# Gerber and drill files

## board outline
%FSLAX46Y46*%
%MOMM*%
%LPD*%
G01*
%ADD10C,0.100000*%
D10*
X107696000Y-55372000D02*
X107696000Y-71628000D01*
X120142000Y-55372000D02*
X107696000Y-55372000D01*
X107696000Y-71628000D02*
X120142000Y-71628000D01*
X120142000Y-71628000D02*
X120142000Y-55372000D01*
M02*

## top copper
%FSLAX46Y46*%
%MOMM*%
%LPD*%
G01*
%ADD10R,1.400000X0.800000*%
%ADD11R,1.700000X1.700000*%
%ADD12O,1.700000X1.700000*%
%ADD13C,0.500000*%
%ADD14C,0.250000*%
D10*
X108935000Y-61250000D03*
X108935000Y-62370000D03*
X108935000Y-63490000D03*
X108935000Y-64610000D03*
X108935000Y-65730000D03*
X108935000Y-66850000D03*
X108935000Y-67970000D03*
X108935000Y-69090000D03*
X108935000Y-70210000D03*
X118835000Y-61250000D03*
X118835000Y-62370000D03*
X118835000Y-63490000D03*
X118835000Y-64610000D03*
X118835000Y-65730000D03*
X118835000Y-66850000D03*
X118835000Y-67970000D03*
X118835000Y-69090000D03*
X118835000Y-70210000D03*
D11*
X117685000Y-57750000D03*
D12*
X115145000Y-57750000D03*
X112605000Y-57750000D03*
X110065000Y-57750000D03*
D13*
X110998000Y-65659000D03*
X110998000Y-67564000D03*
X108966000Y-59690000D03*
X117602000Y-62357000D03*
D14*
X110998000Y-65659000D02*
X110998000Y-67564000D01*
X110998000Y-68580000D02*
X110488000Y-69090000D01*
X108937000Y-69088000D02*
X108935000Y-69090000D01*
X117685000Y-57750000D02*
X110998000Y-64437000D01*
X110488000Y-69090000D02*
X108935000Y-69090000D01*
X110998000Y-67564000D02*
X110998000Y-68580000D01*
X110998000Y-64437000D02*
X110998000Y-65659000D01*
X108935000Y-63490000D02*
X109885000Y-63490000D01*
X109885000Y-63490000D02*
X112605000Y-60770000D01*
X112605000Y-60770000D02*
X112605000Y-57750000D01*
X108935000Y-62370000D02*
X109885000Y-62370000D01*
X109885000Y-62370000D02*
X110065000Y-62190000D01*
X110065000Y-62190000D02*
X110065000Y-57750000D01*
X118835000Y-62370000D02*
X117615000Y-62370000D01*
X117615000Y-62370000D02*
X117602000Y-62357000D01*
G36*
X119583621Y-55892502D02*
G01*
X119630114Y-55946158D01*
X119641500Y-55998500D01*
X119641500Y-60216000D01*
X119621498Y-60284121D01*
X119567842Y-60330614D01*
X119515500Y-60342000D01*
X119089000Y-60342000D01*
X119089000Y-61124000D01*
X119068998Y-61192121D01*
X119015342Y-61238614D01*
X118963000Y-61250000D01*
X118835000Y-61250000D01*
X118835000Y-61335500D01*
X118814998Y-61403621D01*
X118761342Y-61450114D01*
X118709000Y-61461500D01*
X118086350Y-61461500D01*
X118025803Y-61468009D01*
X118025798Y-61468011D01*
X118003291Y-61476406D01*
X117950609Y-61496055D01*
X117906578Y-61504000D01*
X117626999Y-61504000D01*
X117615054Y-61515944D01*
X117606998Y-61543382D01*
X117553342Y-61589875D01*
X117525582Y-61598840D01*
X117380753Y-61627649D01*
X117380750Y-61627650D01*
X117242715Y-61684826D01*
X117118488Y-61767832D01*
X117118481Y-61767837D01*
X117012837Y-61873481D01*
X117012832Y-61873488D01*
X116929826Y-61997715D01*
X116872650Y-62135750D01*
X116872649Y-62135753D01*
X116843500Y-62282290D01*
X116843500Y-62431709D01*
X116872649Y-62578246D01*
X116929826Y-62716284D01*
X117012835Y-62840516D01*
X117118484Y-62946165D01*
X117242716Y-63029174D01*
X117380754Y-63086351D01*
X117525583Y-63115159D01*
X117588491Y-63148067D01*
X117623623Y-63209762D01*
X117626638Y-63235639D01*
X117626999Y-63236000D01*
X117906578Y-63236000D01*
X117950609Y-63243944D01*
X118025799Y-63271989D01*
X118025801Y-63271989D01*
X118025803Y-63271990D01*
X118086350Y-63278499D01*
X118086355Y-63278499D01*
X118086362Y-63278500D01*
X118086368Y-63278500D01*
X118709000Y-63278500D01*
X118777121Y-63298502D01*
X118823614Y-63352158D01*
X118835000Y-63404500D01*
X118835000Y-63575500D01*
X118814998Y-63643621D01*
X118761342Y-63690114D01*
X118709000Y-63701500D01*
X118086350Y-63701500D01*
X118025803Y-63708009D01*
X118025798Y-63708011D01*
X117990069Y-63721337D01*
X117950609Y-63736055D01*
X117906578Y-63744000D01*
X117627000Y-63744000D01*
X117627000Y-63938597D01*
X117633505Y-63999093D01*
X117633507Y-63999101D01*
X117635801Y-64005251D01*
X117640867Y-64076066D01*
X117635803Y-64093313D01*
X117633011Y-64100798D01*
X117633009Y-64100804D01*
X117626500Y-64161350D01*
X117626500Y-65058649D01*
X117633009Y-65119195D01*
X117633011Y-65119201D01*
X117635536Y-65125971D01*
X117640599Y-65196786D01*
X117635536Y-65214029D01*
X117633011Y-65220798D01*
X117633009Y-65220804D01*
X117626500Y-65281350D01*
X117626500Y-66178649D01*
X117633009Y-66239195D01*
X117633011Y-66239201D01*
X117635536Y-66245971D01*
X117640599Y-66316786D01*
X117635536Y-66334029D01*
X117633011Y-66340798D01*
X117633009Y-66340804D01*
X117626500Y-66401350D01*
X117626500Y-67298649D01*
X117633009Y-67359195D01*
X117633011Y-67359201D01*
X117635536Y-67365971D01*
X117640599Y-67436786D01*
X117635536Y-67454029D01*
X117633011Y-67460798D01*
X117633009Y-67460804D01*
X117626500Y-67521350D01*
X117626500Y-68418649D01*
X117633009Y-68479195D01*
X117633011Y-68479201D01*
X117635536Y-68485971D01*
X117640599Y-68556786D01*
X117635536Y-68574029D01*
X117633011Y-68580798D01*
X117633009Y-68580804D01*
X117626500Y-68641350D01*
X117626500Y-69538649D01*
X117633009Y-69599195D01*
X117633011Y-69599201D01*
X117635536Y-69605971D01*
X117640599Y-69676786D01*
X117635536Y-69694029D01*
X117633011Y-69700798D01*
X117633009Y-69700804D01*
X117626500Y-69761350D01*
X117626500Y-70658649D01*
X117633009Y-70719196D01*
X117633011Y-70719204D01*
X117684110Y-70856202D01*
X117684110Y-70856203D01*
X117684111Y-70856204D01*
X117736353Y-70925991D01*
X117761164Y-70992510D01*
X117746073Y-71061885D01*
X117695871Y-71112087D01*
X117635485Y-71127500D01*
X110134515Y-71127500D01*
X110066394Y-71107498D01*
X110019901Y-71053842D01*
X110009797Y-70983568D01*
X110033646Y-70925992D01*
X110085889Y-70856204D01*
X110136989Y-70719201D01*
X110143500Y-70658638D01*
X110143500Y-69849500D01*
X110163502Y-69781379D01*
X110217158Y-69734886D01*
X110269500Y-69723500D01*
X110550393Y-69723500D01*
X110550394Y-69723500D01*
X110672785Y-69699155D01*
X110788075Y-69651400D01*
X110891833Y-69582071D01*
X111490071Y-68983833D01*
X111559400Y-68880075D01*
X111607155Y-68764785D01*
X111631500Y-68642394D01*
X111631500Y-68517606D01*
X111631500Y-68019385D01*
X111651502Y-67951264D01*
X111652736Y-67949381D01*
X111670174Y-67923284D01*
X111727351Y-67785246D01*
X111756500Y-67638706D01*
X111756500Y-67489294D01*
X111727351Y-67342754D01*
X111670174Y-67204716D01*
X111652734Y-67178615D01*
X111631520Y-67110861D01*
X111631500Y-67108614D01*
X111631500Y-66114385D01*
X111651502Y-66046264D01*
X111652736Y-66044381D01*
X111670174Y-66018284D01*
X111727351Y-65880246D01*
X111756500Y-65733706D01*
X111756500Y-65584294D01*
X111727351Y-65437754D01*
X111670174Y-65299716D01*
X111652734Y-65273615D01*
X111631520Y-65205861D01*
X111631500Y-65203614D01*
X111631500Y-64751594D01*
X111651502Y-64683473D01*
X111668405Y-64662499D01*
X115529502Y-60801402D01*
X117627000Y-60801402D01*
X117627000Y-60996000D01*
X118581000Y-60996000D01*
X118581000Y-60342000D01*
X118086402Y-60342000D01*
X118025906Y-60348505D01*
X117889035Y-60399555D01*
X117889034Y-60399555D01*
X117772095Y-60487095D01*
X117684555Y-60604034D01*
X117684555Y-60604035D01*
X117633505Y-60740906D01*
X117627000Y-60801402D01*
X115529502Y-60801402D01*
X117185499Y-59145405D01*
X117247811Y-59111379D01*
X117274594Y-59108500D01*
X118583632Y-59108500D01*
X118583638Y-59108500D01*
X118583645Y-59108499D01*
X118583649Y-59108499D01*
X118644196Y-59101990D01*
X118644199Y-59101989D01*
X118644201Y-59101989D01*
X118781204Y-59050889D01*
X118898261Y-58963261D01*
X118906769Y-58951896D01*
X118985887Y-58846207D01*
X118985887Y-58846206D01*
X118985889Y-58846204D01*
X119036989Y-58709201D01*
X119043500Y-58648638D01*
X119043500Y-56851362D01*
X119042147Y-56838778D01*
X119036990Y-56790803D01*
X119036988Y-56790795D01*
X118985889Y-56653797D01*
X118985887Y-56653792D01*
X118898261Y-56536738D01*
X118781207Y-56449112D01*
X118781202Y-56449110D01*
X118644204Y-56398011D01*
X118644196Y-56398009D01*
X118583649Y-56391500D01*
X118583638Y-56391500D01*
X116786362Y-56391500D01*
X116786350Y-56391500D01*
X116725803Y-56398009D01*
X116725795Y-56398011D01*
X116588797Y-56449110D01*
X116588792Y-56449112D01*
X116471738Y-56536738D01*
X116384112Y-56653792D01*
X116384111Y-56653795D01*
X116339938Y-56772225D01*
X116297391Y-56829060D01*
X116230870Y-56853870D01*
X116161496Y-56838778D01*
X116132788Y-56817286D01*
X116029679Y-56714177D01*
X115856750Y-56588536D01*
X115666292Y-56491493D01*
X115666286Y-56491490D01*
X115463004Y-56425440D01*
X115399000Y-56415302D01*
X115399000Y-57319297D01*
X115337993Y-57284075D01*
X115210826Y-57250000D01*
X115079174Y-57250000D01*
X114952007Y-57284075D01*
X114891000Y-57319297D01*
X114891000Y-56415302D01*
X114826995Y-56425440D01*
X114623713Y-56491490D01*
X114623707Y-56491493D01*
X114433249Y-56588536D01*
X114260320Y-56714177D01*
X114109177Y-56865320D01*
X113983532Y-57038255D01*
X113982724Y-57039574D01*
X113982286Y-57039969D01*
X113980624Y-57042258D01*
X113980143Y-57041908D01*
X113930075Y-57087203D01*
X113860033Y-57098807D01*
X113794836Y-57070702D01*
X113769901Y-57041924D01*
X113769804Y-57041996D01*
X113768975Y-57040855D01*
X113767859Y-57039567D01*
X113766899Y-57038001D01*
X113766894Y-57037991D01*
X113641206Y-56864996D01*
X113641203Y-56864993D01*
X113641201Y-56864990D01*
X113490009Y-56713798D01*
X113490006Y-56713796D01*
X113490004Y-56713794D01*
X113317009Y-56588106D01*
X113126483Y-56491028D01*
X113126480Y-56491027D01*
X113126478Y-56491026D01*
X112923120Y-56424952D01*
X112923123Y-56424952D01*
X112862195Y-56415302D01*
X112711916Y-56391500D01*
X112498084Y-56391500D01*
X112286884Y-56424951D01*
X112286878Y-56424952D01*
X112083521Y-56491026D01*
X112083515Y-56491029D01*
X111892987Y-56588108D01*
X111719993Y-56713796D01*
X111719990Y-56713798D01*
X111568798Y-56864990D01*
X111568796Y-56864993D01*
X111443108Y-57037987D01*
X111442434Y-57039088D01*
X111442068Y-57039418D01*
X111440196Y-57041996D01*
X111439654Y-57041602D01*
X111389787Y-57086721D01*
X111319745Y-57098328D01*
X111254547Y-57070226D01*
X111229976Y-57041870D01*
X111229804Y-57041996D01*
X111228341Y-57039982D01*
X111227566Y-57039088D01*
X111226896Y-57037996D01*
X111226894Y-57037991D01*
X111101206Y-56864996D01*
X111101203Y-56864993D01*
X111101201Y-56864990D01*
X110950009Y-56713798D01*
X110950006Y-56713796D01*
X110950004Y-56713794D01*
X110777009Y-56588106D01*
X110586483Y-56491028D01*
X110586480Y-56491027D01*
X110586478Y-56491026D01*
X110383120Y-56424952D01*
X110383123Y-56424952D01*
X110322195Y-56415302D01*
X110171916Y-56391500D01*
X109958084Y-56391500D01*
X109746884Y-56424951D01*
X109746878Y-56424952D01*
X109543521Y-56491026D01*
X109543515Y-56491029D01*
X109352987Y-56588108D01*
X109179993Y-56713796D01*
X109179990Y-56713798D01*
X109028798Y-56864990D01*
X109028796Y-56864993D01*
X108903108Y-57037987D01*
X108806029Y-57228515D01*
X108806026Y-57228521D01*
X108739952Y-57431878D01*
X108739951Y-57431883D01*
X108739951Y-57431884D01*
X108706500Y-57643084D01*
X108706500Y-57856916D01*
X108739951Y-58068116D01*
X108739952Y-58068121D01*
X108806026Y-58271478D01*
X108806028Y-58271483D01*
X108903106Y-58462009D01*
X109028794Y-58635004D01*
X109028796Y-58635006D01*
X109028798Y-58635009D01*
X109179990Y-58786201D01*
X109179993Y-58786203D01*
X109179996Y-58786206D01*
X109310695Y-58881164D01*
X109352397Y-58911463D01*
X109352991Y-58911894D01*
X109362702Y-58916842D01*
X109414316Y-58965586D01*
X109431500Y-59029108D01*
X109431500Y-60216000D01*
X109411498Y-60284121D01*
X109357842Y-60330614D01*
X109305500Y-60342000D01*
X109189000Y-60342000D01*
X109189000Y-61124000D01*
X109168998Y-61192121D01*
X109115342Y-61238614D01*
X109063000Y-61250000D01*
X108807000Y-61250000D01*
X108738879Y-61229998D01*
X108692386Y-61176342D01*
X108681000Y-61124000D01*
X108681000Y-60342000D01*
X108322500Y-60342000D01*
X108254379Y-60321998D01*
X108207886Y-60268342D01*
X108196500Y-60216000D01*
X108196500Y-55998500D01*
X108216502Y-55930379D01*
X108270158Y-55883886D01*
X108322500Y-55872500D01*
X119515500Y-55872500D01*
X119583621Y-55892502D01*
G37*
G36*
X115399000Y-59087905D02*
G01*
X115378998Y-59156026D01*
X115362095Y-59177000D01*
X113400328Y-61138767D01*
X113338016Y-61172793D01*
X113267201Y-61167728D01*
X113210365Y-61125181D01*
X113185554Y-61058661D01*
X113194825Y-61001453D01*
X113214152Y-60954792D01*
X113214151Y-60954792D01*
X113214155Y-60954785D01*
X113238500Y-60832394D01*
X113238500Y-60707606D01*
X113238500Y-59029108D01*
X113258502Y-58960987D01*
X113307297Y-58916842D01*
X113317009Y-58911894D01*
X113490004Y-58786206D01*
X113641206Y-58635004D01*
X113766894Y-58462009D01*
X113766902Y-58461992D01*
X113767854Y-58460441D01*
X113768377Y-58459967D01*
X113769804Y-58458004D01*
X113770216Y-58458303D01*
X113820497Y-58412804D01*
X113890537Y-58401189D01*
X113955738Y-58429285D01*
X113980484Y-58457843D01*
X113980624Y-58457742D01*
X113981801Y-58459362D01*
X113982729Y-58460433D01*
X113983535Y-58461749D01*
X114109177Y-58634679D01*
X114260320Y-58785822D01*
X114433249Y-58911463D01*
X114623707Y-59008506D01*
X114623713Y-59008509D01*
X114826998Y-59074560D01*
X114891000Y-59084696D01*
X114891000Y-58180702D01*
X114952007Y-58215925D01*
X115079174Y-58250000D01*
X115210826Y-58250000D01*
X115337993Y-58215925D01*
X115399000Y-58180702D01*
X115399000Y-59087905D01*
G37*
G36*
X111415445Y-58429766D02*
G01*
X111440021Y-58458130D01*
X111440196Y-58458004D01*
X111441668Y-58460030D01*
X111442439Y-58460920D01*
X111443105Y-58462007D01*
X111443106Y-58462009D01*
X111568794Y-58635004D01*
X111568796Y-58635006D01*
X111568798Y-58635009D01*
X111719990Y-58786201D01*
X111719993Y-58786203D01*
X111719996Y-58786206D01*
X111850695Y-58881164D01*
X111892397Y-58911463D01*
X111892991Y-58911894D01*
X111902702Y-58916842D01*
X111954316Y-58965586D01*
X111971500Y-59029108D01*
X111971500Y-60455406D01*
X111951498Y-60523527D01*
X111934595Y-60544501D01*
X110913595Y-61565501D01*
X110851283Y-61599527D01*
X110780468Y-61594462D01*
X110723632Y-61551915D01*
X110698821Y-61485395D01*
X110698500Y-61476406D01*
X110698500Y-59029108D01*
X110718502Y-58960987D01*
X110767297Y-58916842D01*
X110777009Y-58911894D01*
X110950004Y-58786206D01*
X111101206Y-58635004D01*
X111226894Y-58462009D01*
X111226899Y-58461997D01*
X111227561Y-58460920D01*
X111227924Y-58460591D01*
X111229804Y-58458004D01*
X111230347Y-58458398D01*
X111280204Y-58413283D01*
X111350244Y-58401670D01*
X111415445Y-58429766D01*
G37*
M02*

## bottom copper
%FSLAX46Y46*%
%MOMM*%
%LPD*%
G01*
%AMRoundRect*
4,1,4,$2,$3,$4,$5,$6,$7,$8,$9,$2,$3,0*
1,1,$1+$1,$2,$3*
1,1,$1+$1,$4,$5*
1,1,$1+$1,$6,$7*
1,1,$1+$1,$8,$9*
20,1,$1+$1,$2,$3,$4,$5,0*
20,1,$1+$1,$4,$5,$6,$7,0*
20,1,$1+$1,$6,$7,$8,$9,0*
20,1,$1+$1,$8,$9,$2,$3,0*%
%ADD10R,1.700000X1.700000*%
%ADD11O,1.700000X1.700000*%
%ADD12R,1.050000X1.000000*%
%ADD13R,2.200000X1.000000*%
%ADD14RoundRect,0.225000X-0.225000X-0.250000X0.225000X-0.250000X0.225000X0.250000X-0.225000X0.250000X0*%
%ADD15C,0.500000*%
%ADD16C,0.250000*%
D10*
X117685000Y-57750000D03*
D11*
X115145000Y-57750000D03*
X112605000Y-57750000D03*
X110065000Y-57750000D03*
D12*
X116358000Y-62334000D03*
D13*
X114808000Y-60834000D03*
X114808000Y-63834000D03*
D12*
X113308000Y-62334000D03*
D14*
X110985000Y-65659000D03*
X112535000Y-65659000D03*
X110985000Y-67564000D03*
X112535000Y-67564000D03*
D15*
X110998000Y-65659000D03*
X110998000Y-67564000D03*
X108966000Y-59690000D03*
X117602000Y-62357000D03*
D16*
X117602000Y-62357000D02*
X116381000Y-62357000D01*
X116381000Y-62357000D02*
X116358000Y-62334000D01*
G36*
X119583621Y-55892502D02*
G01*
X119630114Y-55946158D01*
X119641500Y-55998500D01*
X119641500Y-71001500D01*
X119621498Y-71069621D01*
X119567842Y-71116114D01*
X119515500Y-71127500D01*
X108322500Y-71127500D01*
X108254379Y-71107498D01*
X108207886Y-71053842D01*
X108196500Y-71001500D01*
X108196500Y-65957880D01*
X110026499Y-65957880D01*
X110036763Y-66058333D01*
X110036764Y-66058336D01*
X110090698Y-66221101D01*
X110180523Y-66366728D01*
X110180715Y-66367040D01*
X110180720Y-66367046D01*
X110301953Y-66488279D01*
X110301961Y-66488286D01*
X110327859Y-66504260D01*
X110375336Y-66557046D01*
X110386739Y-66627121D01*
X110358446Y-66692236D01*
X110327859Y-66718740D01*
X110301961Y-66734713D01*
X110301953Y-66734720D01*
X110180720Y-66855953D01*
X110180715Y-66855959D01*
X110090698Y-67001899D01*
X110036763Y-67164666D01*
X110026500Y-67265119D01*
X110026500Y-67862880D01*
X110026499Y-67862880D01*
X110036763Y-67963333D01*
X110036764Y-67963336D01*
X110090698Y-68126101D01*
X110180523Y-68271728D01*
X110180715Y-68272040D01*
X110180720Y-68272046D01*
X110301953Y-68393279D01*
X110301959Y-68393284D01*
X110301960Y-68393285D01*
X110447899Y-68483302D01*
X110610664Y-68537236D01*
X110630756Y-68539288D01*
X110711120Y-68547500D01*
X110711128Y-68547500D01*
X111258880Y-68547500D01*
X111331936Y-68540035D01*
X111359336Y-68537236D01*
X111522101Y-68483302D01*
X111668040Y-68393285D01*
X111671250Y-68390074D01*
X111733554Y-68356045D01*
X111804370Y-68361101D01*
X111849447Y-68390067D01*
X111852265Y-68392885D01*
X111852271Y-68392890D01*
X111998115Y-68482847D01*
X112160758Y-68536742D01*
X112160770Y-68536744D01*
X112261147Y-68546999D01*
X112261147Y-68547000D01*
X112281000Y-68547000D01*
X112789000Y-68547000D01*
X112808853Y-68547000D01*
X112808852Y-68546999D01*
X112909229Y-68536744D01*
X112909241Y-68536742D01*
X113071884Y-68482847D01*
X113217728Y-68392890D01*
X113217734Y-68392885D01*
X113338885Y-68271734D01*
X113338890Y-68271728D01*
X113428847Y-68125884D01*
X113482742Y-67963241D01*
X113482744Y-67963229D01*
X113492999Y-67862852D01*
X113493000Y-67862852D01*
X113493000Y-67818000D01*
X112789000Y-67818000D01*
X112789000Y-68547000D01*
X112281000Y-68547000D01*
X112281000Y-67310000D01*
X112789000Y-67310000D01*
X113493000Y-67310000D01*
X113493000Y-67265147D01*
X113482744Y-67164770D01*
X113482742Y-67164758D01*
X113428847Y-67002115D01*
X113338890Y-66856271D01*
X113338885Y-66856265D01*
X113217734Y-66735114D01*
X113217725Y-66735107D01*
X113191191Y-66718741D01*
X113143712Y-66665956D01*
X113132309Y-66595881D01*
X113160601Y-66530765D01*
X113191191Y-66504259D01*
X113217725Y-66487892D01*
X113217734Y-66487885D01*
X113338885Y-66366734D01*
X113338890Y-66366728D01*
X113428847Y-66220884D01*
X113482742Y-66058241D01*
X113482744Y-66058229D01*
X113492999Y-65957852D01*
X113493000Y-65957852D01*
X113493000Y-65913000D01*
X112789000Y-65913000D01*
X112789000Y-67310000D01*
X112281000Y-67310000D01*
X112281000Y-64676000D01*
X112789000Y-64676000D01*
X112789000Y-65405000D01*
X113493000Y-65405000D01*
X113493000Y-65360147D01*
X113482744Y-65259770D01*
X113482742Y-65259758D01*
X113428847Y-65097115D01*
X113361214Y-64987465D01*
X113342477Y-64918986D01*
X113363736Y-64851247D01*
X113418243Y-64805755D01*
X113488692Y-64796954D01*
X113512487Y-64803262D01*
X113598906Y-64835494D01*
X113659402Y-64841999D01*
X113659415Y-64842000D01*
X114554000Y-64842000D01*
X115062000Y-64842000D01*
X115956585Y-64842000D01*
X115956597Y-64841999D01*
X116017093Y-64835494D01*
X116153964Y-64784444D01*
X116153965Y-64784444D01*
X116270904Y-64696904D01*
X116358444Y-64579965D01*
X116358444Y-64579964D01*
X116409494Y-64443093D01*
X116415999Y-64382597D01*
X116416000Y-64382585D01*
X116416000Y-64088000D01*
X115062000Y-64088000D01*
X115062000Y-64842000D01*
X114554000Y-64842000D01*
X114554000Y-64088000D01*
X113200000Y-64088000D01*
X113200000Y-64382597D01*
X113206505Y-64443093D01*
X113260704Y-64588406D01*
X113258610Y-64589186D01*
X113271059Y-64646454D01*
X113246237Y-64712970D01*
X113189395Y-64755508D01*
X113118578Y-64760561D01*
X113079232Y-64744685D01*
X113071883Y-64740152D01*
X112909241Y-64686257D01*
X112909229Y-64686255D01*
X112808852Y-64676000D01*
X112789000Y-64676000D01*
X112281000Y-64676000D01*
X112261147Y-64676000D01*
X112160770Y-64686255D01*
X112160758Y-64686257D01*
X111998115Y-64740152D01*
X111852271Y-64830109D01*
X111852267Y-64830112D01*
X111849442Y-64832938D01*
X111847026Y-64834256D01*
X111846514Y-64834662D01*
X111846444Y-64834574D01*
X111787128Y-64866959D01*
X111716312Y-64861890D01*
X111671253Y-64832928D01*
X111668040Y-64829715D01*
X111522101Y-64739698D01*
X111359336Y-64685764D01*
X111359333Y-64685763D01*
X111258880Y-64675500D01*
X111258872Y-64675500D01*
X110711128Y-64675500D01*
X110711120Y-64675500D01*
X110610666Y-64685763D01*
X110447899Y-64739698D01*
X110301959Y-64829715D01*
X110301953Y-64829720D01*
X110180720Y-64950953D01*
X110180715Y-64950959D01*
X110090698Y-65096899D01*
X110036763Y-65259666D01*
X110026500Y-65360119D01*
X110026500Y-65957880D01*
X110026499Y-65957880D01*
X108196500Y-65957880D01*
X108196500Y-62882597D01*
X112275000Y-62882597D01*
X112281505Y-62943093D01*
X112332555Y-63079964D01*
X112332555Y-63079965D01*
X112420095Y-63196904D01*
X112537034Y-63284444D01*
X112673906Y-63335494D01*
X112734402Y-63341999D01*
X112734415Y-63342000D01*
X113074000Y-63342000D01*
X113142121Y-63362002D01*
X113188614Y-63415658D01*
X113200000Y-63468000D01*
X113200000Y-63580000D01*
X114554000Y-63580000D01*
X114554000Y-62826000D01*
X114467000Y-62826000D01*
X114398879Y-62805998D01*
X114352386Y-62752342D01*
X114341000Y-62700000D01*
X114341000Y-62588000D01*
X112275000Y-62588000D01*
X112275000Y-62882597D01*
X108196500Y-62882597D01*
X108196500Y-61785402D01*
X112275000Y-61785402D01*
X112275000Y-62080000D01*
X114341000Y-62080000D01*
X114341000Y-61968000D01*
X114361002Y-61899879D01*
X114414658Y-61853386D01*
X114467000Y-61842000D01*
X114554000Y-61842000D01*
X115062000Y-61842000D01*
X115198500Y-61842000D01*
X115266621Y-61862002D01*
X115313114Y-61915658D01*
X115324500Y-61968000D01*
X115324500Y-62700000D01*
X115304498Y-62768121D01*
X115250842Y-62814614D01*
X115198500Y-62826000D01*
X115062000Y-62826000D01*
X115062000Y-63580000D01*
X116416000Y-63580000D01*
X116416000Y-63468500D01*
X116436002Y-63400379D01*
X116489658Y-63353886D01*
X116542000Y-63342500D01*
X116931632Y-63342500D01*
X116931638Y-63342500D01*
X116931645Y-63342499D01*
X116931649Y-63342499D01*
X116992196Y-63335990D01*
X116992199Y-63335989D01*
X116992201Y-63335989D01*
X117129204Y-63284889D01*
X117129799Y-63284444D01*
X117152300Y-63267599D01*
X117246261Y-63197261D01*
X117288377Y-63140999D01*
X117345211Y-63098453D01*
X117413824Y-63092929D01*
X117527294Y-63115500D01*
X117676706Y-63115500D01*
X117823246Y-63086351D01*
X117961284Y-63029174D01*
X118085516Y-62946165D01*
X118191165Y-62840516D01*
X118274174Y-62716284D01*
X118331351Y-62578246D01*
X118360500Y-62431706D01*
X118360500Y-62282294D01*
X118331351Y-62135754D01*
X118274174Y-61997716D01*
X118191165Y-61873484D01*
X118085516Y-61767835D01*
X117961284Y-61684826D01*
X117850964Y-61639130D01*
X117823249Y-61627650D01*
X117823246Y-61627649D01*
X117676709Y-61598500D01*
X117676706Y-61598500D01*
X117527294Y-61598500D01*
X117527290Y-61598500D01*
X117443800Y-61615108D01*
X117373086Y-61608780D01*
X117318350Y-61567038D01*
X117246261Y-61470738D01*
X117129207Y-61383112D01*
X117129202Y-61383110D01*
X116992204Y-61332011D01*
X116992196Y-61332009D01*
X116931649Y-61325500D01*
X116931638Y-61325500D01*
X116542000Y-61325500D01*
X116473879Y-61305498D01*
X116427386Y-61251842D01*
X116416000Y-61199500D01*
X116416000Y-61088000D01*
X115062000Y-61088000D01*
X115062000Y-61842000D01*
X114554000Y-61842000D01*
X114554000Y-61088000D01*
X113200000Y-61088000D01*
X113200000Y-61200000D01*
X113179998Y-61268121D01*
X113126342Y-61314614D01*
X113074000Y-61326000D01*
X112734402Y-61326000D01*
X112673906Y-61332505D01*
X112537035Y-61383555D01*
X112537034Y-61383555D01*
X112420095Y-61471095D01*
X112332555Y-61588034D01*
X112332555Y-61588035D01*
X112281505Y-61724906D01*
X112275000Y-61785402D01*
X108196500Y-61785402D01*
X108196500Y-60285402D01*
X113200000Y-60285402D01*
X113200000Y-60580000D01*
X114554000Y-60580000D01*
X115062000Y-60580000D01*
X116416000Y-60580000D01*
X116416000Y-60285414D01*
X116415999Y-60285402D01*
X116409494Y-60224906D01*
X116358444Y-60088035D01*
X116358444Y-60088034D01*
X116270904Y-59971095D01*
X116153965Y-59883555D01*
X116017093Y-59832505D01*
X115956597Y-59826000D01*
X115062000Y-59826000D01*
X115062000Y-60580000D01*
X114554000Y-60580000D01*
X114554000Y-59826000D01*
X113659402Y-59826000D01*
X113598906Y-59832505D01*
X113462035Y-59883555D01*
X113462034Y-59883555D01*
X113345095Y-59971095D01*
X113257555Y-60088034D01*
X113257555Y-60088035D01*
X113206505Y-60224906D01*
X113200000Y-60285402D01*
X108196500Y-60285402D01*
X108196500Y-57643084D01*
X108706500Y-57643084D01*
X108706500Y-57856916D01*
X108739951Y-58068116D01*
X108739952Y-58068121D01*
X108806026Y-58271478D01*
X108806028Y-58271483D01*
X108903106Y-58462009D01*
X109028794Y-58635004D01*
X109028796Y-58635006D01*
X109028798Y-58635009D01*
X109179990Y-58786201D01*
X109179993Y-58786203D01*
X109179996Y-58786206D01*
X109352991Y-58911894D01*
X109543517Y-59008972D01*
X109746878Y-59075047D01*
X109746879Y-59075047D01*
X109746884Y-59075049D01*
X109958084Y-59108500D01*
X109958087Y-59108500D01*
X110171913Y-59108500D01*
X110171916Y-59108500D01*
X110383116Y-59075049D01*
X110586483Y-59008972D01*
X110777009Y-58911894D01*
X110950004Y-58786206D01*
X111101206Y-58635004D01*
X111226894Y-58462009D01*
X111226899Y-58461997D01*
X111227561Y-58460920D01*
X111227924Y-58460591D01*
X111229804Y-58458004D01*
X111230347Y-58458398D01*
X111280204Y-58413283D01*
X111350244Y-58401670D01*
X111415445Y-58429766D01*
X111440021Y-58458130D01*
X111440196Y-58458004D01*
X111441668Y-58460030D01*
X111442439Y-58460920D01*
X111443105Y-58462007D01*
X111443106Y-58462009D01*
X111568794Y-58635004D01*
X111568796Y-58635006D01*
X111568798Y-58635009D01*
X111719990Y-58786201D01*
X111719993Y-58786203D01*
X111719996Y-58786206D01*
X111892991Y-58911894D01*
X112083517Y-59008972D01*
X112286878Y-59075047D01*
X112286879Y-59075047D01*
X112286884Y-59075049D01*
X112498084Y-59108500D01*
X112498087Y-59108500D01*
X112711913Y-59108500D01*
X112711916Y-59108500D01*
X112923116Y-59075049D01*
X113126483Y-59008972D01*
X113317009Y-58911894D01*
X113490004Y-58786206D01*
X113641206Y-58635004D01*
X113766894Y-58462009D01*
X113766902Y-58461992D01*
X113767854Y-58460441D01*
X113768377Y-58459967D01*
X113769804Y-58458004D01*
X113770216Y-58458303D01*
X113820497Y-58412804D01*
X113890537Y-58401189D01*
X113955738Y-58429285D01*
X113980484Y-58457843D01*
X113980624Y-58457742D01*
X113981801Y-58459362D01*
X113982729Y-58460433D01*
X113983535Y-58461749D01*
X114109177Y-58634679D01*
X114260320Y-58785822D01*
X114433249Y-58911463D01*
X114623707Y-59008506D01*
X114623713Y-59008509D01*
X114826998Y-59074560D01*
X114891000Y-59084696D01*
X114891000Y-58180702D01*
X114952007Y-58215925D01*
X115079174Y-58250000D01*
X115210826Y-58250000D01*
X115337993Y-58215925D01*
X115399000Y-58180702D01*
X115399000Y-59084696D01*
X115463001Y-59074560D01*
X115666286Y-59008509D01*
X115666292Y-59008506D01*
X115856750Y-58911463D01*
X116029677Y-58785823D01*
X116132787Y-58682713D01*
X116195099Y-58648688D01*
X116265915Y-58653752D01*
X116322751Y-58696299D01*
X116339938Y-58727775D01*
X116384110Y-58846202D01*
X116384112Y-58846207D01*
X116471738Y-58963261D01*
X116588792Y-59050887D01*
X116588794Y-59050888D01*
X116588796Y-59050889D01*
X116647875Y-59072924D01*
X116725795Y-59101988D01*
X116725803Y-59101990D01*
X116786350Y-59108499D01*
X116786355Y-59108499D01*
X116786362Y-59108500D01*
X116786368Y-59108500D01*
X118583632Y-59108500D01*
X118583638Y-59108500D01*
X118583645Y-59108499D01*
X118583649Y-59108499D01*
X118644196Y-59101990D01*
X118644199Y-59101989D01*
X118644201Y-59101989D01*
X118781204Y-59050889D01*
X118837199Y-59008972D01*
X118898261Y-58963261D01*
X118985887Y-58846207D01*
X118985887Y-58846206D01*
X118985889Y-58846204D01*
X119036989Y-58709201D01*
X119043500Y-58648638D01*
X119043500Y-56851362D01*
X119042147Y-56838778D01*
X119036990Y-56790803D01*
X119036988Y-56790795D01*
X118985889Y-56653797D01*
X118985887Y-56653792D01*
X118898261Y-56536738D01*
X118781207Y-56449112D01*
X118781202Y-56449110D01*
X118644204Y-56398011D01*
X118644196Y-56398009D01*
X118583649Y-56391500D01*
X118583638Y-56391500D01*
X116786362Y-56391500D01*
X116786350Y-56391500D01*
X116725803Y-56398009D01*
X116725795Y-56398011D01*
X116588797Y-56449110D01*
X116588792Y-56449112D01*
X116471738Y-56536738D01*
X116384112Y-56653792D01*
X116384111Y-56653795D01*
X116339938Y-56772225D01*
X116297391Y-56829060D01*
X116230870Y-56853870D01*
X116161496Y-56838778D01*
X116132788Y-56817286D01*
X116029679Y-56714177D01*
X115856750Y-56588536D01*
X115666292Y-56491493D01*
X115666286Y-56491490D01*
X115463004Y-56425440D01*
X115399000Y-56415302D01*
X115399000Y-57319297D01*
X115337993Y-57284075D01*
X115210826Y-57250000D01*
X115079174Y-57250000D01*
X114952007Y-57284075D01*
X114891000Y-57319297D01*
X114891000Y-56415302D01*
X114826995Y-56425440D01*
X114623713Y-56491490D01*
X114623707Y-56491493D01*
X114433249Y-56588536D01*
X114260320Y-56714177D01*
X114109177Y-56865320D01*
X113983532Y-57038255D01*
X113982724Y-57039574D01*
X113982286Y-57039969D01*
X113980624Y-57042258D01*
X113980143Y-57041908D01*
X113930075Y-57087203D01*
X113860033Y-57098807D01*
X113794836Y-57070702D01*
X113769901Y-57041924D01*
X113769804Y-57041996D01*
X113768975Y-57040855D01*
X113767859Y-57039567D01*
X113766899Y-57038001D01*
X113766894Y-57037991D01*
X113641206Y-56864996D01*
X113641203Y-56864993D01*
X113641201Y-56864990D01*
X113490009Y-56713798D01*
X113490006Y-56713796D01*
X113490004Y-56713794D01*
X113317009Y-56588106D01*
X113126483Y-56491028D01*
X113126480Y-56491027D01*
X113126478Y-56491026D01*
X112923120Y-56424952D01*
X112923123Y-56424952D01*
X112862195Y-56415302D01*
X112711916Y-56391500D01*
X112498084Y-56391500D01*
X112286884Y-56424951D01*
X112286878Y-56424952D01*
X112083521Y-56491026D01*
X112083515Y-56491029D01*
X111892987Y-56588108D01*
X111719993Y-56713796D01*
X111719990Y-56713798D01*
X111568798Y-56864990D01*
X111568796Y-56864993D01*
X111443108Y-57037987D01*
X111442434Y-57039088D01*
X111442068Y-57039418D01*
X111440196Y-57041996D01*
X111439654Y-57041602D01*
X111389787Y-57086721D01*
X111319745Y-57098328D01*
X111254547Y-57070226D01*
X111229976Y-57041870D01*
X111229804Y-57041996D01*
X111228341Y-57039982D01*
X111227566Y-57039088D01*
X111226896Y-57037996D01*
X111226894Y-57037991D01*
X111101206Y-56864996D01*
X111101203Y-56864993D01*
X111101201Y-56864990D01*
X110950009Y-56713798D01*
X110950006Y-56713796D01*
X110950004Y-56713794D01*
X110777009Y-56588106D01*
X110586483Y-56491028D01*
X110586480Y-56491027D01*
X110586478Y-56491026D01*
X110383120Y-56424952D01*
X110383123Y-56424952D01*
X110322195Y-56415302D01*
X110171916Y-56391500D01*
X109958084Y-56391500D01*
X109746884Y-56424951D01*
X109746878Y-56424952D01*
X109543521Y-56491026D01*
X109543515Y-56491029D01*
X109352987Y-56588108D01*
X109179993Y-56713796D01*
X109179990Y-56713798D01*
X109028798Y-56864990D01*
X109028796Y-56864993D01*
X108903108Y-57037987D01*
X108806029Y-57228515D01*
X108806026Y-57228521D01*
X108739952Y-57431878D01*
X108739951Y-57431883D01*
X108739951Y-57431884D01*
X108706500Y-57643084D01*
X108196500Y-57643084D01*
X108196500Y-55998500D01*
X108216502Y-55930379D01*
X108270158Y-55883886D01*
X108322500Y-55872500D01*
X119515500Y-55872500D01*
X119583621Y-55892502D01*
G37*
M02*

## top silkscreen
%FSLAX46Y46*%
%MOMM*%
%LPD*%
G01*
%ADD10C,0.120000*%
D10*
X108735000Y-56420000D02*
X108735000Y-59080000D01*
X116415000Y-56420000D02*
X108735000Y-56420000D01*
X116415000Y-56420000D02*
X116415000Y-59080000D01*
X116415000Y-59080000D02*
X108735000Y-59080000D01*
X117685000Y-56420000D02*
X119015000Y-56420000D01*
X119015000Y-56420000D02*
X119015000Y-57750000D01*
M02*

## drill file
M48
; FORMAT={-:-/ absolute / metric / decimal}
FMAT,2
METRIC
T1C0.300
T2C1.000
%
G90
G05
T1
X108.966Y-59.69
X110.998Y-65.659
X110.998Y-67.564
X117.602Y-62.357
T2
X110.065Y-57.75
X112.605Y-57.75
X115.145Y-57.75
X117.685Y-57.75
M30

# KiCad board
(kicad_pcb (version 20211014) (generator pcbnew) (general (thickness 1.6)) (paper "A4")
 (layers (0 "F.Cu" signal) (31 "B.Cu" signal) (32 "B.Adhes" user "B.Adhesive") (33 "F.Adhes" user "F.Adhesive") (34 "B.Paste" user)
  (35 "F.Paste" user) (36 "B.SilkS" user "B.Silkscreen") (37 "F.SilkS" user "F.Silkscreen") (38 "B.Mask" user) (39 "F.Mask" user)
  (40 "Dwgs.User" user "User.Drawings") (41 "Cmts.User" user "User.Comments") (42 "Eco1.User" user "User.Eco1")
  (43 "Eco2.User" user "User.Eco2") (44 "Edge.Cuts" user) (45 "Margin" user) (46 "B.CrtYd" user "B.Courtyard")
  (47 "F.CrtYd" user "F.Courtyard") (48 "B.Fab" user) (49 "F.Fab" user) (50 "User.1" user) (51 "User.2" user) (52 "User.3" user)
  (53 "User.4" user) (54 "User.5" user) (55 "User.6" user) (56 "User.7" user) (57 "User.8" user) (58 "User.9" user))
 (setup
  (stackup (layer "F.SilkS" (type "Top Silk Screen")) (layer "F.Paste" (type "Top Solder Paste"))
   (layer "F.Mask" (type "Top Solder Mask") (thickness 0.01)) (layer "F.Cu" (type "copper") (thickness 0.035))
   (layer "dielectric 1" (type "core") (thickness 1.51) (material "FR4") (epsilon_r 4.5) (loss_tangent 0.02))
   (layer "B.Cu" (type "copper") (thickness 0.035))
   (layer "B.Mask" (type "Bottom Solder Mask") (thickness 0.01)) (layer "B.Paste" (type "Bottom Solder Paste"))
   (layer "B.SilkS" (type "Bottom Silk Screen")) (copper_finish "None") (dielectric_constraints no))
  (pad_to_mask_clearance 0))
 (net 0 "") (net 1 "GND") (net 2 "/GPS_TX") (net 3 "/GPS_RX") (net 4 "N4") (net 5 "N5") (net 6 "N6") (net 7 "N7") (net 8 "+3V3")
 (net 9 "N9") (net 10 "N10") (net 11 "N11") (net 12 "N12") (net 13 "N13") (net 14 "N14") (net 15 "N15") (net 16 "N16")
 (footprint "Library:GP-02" (layer "F.Cu") (at 114.135 65.75)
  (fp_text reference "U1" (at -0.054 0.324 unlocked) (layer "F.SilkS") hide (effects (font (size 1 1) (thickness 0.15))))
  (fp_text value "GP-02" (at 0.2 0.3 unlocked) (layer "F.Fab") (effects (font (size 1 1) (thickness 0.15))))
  (pad "1" smd rect (at -5.2 -4.5) (size 1.4 0.8) (layers "F.Cu" "F.Paste" "F.Mask") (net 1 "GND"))
  (pad "2" smd rect (at -5.2 -3.38) (size 1.4 0.8) (layers "F.Cu" "F.Paste" "F.Mask") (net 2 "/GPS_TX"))
  (pad "3" smd rect (at -5.2 -2.26) (size 1.4 0.8) (layers "F.Cu" "F.Paste" "F.Mask") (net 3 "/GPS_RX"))
  (pad "4" smd rect (at -5.2 -1.14) (size 1.4 0.8) (layers "F.Cu" "F.Paste" "F.Mask") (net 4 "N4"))
  (pad "5" smd rect (at -5.2 -0.02) (size 1.4 0.8) (layers "F.Cu" "F.Paste" "F.Mask") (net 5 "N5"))
  (pad "6" smd rect (at -5.2 1.1) (size 1.4 0.8) (layers "F.Cu" "F.Paste" "F.Mask") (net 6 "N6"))
  (pad "7" smd rect (at -5.2 2.22) (size 1.4 0.8) (layers "F.Cu" "F.Paste" "F.Mask") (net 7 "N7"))
  (pad "8" smd rect (at -5.2 3.34) (size 1.4 0.8) (layers "F.Cu" "F.Paste" "F.Mask") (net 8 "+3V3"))
  (pad "9" smd rect (at -5.2 4.46) (size 1.4 0.8) (layers "F.Cu" "F.Paste" "F.Mask") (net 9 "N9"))
  (pad "10" smd rect (at 4.7 -4.5) (size 1.4 0.8) (layers "F.Cu" "F.Paste" "F.Mask") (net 1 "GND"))
  (pad "11" smd rect (at 4.7 -3.38) (size 1.4 0.8) (layers "F.Cu" "F.Paste" "F.Mask") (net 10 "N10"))
  (pad "12" smd rect (at 4.7 -2.26) (size 1.4 0.8) (layers "F.Cu" "F.Paste" "F.Mask") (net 1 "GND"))
  (pad "13" smd rect (at 4.7 -1.14) (size 1.4 0.8) (layers "F.Cu" "F.Paste" "F.Mask") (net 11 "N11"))
  (pad "14" smd rect (at 4.7 -0.02) (size 1.4 0.8) (layers "F.Cu" "F.Paste" "F.Mask") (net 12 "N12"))
  (pad "15" smd rect (at 4.7 1.1) (size 1.4 0.8) (layers "F.Cu" "F.Paste" "F.Mask") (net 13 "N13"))
  (pad "16" smd rect (at 4.7 2.22) (size 1.4 0.8) (layers "F.Cu" "F.Paste" "F.Mask") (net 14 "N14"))
  (pad "17" smd rect (at 4.7 3.34) (size 1.4 0.8) (layers "F.Cu" "F.Paste" "F.Mask") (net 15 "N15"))
  (pad "18" smd rect (at 4.7 4.46) (size 1.4 0.8) (layers "F.Cu" "F.Paste" "F.Mask") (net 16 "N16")))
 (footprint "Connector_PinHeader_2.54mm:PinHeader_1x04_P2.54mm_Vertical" (layer "F.Cu") (at 117.685 57.75 -90)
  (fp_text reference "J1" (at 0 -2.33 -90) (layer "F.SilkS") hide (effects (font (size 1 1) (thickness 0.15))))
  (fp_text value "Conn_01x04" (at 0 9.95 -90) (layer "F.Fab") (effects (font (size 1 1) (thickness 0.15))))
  (fp_line (start -1.33 8.95) (end 1.33 8.95) (layer "F.SilkS") (width 0.12))
  (fp_line (start -1.33 1.27) (end -1.33 8.95) (layer "F.SilkS") (width 0.12))
  (fp_line (start -1.33 1.27) (end 1.33 1.27) (layer "F.SilkS") (width 0.12))
  (fp_line (start 1.33 1.27) (end 1.33 8.95) (layer "F.SilkS") (width 0.12))
  (fp_line (start -1.33 0) (end -1.33 -1.33) (layer "F.SilkS") (width 0.12))
  (fp_line (start -1.33 -1.33) (end 0 -1.33) (layer "F.SilkS") (width 0.12))
  (pad "1" thru_hole rect (at 0 0 270) (size 1.7 1.7) (drill 1) (layers *.Cu *.Mask) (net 8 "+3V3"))
  (pad "2" thru_hole oval (at 0 2.54 270) (size 1.7 1.7) (drill 1) (layers *.Cu *.Mask) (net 1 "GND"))
  (pad "3" thru_hole oval (at 0 5.08 270) (size 1.7 1.7) (drill 1) (layers *.Cu *.Mask) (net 3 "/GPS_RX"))
  (pad "4" thru_hole oval (at 0 7.62 270) (size 1.7 1.7) (drill 1) (layers *.Cu *.Mask) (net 2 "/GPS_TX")))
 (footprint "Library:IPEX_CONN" (layer "B.Cu") (at 114.808 62.334 -90)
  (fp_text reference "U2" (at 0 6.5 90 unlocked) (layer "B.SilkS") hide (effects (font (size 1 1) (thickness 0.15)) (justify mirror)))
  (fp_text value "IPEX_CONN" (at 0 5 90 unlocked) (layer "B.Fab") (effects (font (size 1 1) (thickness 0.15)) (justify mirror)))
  (pad "1" smd rect (at 0 -1.55 270) (size 1 1.05) (layers "B.Cu" "B.Paste" "B.Mask") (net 10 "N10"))
  (pad "2" smd rect (at -1.5 0 270) (size 1 2.2) (layers "B.Cu" "B.Paste" "B.Mask") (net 1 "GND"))
  (pad "3" smd rect (at 1.5 0 270) (size 1 2.2) (layers "B.Cu" "B.Paste" "B.Mask") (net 1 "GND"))
  (pad "4" smd rect (at 0 1.5 270) (size 1 1.05) (layers "B.Cu" "B.Paste" "B.Mask") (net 1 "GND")))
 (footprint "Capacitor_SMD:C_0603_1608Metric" (layer "B.Cu") (at 111.76 65.659)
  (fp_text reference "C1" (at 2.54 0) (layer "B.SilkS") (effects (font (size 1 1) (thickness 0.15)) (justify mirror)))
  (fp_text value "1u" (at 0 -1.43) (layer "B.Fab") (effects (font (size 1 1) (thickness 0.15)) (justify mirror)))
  (pad "1" smd roundrect (at -0.775 0) (size 0.9 0.95) (layers "B.Cu" "B.Paste" "B.Mask") (roundrect_rratio 0.25) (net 8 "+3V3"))
  (pad "2" smd roundrect (at 0.775 0) (size 0.9 0.95) (layers "B.Cu" "B.Paste" "B.Mask") (roundrect_rratio 0.25) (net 1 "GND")))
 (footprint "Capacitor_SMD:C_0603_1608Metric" (layer "B.Cu") (at 111.76 67.564)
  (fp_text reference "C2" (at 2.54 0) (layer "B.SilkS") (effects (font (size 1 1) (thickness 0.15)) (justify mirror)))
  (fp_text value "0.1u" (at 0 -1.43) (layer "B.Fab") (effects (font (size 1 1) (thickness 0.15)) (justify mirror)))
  (pad "1" smd roundrect (at -0.775 0) (size 0.9 0.95) (layers "B.Cu" "B.Paste" "B.Mask") (roundrect_rratio 0.25) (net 8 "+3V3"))
  (pad "2" smd roundrect (at 0.775 0) (size 0.9 0.95) (layers "B.Cu" "B.Paste" "B.Mask") (roundrect_rratio 0.25) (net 1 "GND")))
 (gr_line (start 107.696 55.372) (end 107.696 71.628) (layer "Edge.Cuts") (width 0.1))
 (gr_line (start 120.142 55.372) (end 107.696 55.372) (layer "Edge.Cuts") (width 0.1))
 (gr_line (start 107.696 71.628) (end 120.142 71.628) (layer "Edge.Cuts") (width 0.1))
 (gr_line (start 120.142 71.628) (end 120.142 55.372) (layer "Edge.Cuts") (width 0.1))
 (segment (start 110.998 65.659) (end 110.998 67.564) (width 0.25) (layer "F.Cu") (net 8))
 (segment (start 110.998 68.58) (end 110.488 69.09) (width 0.25) (layer "F.Cu") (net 8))
 (segment (start 108.937 69.088) (end 108.935 69.09) (width 0.25) (layer "F.Cu") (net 8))
 (segment (start 117.685 57.75) (end 110.998 64.437) (width 0.25) (layer "F.Cu") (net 8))
 (segment (start 110.488 69.09) (end 108.935 69.09) (width 0.25) (layer "F.Cu") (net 8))
 (segment (start 110.998 67.564) (end 110.998 68.58) (width 0.25) (layer "F.Cu") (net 8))
 (segment (start 110.998 64.437) (end 110.998 65.659) (width 0.25) (layer "F.Cu") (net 8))
 (via (at 110.998 65.659) (size 0.5) (drill 0.3) (layers "F.Cu" "B.Cu") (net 8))
 (via (at 110.998 67.564) (size 0.5) (drill 0.3) (layers "F.Cu" "B.Cu") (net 8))
 (via (at 108.966 59.69) (size 0.5) (drill 0.3) (layers "F.Cu" "B.Cu") (free) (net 1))
 (segment (start 108.935 63.49) (end 109.885 63.49) (width 0.25) (layer "F.Cu") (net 3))
 (segment (start 109.885 63.49) (end 112.605 60.77) (width 0.25) (layer "F.Cu") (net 3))
 (segment (start 112.605 60.77) (end 112.605 57.75) (width 0.25) (layer "F.Cu") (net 3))
 (segment (start 108.935 62.37) (end 109.885 62.37) (width 0.25) (layer "F.Cu") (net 2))
 (segment (start 109.885 62.37) (end 110.065 62.19) (width 0.25) (layer "F.Cu") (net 2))
 (segment (start 110.065 62.19) (end 110.065 57.75) (width 0.25) (layer "F.Cu") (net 2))
 (segment (start 118.835 62.37) (end 117.615 62.37) (width 0.25) (layer "F.Cu") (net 10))
 (segment (start 117.615 62.37) (end 117.602 62.357) (width 0.25) (layer "F.Cu") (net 10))
 (via (at 117.602 62.357) (size 0.5) (drill 0.3) (layers "F.Cu" "B.Cu") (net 10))
 (segment (start 117.602 62.357) (end 116.381 62.357) (width 0.25) (layer "B.Cu") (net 10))
 (segment (start 116.381 62.357) (end 116.358 62.334) (width 0.25) (layer "B.Cu") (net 10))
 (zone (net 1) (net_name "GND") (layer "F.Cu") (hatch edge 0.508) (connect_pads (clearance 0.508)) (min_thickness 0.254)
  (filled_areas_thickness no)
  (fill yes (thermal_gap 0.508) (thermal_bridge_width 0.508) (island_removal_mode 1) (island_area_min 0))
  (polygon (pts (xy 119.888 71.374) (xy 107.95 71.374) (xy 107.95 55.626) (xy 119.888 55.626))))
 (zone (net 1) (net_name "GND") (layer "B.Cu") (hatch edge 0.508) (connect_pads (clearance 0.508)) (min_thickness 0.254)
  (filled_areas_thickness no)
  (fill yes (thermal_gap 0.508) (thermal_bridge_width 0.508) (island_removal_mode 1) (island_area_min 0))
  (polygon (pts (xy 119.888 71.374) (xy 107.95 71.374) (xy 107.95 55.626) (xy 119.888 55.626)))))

